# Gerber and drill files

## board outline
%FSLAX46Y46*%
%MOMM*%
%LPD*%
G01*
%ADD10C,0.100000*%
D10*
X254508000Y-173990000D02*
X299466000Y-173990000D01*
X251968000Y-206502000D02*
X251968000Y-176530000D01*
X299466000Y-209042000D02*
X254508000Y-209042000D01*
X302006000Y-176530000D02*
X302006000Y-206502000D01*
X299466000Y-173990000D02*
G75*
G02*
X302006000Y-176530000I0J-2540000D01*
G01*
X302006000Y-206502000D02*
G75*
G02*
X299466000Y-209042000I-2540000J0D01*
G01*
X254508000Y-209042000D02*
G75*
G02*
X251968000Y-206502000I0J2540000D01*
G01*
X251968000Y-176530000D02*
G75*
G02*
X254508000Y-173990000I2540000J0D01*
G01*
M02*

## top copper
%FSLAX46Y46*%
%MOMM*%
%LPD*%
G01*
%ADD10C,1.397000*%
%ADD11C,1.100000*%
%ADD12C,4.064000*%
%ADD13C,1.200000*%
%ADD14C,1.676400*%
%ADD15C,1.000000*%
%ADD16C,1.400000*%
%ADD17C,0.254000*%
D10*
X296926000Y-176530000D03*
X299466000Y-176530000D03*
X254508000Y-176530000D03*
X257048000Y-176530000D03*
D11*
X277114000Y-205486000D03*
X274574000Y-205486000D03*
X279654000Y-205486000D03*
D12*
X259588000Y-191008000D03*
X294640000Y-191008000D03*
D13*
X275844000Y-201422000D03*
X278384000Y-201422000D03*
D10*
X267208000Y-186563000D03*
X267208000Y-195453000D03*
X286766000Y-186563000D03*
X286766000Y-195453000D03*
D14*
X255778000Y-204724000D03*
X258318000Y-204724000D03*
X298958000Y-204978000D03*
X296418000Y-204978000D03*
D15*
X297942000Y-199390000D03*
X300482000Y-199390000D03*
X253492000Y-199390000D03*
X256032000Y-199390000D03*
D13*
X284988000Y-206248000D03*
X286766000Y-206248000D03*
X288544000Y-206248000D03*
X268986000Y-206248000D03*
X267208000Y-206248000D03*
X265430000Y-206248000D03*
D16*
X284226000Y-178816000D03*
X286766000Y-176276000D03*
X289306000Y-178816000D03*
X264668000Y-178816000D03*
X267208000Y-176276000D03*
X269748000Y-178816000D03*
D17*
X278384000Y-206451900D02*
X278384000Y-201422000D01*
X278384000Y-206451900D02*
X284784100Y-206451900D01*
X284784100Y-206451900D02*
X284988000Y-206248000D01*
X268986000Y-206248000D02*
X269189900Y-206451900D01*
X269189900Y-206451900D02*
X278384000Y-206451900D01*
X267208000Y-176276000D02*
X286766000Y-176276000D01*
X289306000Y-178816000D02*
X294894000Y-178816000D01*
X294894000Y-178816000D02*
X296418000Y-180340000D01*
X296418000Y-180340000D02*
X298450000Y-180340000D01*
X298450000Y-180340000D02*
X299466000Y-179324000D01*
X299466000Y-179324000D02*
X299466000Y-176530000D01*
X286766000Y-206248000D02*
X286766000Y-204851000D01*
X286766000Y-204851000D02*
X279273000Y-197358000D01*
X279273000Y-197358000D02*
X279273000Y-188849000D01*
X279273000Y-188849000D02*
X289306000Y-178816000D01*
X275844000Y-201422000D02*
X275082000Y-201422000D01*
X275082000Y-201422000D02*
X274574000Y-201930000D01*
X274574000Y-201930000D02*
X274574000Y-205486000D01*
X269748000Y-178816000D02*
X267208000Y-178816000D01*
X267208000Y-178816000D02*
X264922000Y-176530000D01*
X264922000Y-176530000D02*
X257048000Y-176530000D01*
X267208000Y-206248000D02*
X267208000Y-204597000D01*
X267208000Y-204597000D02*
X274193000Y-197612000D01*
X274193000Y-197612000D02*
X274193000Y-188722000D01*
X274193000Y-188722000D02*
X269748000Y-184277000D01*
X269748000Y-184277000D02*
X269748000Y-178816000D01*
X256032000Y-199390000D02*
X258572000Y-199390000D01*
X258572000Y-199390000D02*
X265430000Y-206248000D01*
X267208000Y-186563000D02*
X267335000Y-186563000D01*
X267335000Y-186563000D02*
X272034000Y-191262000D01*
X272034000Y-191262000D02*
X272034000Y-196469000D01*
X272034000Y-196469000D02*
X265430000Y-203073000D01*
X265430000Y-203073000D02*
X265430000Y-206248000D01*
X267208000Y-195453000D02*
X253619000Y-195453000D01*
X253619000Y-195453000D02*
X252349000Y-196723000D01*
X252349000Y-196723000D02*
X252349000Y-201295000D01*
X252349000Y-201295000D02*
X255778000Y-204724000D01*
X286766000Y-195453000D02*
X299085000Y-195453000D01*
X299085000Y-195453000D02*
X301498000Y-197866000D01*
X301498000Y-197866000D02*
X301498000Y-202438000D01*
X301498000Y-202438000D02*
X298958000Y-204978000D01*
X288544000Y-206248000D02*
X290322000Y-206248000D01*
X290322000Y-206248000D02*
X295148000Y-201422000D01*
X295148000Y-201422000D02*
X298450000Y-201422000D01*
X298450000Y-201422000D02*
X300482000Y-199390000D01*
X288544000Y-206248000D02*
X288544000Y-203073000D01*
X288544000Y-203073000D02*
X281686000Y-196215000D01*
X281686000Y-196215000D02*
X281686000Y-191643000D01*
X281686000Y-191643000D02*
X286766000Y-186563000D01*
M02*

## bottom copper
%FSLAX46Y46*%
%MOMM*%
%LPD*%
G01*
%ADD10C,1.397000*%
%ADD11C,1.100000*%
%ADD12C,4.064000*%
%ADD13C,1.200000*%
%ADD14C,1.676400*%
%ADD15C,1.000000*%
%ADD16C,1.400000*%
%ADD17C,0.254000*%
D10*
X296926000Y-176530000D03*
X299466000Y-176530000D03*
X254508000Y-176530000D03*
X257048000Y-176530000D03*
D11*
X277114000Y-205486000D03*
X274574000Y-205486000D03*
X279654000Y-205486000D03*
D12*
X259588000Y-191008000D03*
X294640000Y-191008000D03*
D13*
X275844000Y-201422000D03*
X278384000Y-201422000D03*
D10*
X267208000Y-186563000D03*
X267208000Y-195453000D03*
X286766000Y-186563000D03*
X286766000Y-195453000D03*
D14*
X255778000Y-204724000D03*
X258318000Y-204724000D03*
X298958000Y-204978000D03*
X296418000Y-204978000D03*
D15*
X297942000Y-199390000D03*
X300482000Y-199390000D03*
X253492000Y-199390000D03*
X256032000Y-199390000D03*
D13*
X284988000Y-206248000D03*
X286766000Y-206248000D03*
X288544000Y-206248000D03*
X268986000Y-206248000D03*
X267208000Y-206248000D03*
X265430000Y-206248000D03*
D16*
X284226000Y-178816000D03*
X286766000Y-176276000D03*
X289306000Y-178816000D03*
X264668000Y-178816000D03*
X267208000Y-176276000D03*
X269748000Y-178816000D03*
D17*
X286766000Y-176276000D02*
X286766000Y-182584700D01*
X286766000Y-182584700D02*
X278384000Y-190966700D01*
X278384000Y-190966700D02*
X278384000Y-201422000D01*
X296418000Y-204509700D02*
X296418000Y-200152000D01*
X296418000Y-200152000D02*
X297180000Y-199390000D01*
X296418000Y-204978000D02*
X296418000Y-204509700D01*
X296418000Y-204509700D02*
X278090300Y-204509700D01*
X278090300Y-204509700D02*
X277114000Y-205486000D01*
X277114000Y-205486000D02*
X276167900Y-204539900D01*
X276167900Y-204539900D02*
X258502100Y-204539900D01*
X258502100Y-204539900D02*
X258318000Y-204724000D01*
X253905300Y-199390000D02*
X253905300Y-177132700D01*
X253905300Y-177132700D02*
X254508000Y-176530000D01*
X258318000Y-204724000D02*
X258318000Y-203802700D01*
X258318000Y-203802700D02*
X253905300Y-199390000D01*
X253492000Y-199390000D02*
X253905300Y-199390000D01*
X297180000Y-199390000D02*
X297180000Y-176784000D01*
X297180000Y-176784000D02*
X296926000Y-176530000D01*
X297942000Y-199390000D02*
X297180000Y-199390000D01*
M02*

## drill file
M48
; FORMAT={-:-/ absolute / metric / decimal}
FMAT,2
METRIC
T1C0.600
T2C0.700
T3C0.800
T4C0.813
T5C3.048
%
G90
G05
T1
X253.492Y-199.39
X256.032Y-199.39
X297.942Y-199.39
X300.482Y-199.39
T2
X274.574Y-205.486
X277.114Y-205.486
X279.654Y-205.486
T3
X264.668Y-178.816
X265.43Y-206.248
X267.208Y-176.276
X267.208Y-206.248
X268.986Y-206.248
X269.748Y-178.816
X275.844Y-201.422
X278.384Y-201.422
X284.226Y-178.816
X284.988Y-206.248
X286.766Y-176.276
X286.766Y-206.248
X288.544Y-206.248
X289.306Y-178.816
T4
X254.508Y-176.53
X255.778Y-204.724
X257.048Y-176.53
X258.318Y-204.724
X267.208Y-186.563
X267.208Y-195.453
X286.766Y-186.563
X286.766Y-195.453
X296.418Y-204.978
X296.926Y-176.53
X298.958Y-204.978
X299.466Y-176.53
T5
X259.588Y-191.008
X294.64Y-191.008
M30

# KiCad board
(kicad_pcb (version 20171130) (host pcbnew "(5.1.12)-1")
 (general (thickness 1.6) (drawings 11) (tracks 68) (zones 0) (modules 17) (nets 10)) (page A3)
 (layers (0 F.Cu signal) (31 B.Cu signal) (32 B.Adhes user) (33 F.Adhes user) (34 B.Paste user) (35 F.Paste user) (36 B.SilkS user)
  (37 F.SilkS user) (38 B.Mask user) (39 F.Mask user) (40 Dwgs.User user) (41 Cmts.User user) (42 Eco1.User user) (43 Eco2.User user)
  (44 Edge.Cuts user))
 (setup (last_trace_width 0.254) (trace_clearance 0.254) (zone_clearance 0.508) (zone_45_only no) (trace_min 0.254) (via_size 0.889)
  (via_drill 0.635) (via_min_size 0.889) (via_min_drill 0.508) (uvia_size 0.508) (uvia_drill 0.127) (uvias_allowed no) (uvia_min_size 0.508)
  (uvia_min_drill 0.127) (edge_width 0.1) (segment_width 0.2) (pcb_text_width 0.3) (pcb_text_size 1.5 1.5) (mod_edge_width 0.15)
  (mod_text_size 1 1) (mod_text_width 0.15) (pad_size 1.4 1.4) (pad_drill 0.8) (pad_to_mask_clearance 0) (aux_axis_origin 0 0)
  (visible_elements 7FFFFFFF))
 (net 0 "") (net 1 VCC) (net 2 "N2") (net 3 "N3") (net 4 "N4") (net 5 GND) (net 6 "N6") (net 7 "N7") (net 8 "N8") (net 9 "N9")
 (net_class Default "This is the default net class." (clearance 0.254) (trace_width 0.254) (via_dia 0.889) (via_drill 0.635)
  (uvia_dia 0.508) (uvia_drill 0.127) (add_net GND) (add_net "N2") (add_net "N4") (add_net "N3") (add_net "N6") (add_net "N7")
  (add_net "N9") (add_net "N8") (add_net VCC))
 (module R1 (layer F.Cu) (at 298.196 176.53) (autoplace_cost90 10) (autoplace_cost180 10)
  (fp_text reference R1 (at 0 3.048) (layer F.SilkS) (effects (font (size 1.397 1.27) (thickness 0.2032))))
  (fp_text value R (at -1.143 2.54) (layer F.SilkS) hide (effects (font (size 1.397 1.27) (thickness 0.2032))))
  (pad 1 thru_hole circle (at -1.27 0) (size 1.397 1.397) (drill 0.8128) (layers *.Cu *.Mask F.SilkS) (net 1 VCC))
  (pad 2 thru_hole circle (at 1.27 0) (size 1.397 1.397) (drill 0.8128) (layers *.Cu *.Mask F.SilkS) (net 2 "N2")))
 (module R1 (layer F.Cu) (at 255.778 176.53) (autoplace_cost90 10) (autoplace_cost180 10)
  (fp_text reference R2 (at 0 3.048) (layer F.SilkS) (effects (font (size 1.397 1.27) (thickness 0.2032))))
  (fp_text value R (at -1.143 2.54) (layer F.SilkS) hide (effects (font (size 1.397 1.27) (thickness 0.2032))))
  (pad 1 thru_hole circle (at -1.27 0) (size 1.397 1.397) (drill 0.8128) (layers *.Cu *.Mask F.SilkS) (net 1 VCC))
  (pad 2 thru_hole circle (at 1.27 0) (size 1.397 1.397) (drill 0.8128) (layers *.Cu *.Mask F.SilkS) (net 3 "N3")))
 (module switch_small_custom (layer F.Cu) (at 277.114 205.486)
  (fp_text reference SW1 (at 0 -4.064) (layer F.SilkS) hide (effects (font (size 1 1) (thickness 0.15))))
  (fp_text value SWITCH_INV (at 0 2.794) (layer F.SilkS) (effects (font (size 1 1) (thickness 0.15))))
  (pad 2 thru_hole circle (at 0 0) (size 1.1 1.1) (drill 0.7) (layers *.Cu *.Mask F.SilkS) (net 1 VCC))
  (pad 1 thru_hole circle (at -2.54 0) (size 1.1 1.1) (drill 0.7) (layers *.Cu *.Mask F.SilkS) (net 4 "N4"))
  (pad 3 thru_hole circle (at 2.54 0) (size 1.1 1.1) (drill 0.7) (layers *.Cu *.Mask F.SilkS)))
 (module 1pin (layer F.Cu) (at 259.588 191.008)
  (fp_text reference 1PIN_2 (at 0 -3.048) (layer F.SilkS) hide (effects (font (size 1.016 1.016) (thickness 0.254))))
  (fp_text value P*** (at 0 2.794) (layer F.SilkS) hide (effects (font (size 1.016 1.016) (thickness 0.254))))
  (pad 1 thru_hole circle (at 0 0) (size 4.064 4.064) (drill 3.048) (layers *.Cu *.Mask F.SilkS)))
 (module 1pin (layer F.Cu) (at 294.64 191.008)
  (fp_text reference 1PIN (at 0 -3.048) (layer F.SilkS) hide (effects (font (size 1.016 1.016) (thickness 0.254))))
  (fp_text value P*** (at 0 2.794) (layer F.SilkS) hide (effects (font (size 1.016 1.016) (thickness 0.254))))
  (pad 1 thru_hole circle (at 0 0) (size 4.064 4.064) (drill 3.048) (layers *.Cu *.Mask F.SilkS)))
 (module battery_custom (layer F.Cu) (at 277.114 201.422)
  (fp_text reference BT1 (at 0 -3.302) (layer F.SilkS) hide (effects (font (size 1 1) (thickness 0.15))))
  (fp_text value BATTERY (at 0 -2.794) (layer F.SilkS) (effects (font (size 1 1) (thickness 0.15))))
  (pad 1 thru_hole circle (at -1.27 0) (size 1.2 1.2) (drill 0.8) (layers *.Cu *.Mask F.SilkS) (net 4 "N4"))
  (pad 2 thru_hole circle (at 1.27 0) (size 1.2 1.2) (drill 0.8) (layers *.Cu *.Mask F.SilkS) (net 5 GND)))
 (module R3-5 (layer F.Cu) (at 267.208 191.008 270)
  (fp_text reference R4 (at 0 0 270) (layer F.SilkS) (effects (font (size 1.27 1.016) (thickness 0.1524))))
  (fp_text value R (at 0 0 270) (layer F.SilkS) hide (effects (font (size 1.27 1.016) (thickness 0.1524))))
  (pad 1 thru_hole circle (at -4.445 0 270) (size 1.397 1.397) (drill 0.8128) (layers *.Cu *.Mask F.SilkS) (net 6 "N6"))
  (pad 2 thru_hole circle (at 4.445 0 270) (size 1.397 1.397) (drill 0.8128) (layers *.Cu *.Mask F.SilkS) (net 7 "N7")))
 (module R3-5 (layer F.Cu) (at 286.766 191.008 270)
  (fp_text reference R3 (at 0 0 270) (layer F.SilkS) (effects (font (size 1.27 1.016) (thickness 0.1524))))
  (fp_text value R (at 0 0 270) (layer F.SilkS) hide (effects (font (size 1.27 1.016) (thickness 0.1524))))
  (pad 1 thru_hole circle (at -4.445 0 270) (size 1.397 1.397) (drill 0.8128) (layers *.Cu *.Mask F.SilkS) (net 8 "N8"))
  (pad 2 thru_hole circle (at 4.445 0 270) (size 1.397 1.397) (drill 0.8128) (layers *.Cu *.Mask F.SilkS) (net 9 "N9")))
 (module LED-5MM (layer F.Cu) (at 257.048 204.724)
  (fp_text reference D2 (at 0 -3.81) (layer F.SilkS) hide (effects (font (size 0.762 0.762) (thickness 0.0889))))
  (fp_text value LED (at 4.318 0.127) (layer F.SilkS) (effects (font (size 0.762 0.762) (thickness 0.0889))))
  (pad 1 thru_hole circle (at -1.27 0) (size 1.6764 1.6764) (drill 0.8128) (layers *.Cu *.Mask F.SilkS) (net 7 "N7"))
  (pad 2 thru_hole circle (at 1.27 0) (size 1.6764 1.6764) (drill 0.8128) (layers *.Cu *.Mask F.SilkS) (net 1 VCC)))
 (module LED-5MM (layer F.Cu) (at 297.688 204.978 180)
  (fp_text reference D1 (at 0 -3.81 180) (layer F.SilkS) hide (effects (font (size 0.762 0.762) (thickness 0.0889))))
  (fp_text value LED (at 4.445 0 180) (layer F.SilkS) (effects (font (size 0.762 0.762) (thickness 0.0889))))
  (pad 1 thru_hole circle (at -1.27 0 180) (size 1.6764 1.6764) (drill 0.8128) (layers *.Cu *.Mask F.SilkS) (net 9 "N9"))
  (pad 2 thru_hole circle (at 1.27 0 180) (size 1.6764 1.6764) (drill 0.8128) (layers *.Cu *.Mask F.SilkS) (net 1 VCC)))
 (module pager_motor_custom (layer F.Cu) (at 299.212 199.39)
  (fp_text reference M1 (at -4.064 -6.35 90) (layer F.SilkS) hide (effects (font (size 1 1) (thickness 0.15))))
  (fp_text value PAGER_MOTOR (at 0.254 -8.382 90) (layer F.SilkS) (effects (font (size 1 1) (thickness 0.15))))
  (pad 1 thru_hole circle (at -1.27 0) (size 1 1) (drill 0.6) (layers *.Cu *.Mask F.SilkS) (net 1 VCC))
  (pad 2 thru_hole circle (at 1.27 0) (size 1 1) (drill 0.6) (layers *.Cu *.Mask F.SilkS) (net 8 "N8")))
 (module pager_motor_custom (layer F.Cu) (at 254.762 199.39)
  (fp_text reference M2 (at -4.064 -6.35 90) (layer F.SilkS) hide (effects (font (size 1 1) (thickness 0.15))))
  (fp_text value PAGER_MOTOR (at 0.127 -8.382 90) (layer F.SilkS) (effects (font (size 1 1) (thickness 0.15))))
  (pad 1 thru_hole circle (at -1.27 0) (size 1 1) (drill 0.6) (layers *.Cu *.Mask F.SilkS) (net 1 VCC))
  (pad 2 thru_hole circle (at 1.27 0) (size 1 1) (drill 0.6) (layers *.Cu *.Mask F.SilkS) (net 6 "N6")))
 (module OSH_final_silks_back (layer F.Cu) (at 277.114 178.943)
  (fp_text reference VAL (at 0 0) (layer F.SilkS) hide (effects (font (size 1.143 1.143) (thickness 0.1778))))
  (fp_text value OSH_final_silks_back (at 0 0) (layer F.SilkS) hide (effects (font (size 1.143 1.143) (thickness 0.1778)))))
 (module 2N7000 (layer F.Cu) (at 286.766 206.248)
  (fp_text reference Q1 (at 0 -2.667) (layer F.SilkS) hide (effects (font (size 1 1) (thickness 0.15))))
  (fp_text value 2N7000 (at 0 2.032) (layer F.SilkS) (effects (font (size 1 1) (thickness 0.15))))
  (pad 1 thru_hole circle (at -1.778 0) (size 1.2 1.2) (drill 0.8) (layers *.Cu *.Mask F.SilkS) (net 5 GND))
  (pad 2 thru_hole circle (at 0 0) (size 1.2 1.2) (drill 0.8) (layers *.Cu *.Mask F.SilkS) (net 2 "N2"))
  (pad 3 thru_hole circle (at 1.778 0) (size 1.2 1.2) (drill 0.8) (layers *.Cu *.Mask F.SilkS) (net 8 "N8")))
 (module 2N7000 (layer F.Cu) (at 267.208 206.248 180)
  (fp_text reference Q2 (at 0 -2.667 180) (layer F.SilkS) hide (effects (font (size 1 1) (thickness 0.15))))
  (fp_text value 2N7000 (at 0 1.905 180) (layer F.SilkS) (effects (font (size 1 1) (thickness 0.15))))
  (pad 1 thru_hole circle (at -1.778 0 180) (size 1.2 1.2) (drill 0.8) (layers *.Cu *.Mask F.SilkS) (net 5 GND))
  (pad 2 thru_hole circle (at 0 0 180) (size 1.2 1.2) (drill 0.8) (layers *.Cu *.Mask F.SilkS) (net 3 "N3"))
  (pad 3 thru_hole circle (at 1.778 0 180) (size 1.2 1.2) (drill 0.8) (layers *.Cu *.Mask F.SilkS) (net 6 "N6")))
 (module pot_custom (layer F.Cu) (at 286.766 178.816)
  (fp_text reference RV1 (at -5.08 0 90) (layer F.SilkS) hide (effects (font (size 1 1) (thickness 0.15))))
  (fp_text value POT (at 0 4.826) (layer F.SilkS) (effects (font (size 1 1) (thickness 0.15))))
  (pad 1 thru_hole circle (at -2.54 0) (size 1.4 1.4) (drill 0.8) (layers *.Cu *.Mask F.SilkS))
  (pad 2 thru_hole circle (at 0 -2.54) (size 1.4 1.4) (drill 0.8) (layers *.Cu *.Mask F.SilkS) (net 5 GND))
  (pad 3 thru_hole circle (at 2.54 0) (size 1.4 1.4) (drill 0.8) (layers *.Cu *.Mask F.SilkS) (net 2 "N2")))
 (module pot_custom (layer F.Cu) (at 267.208 178.816)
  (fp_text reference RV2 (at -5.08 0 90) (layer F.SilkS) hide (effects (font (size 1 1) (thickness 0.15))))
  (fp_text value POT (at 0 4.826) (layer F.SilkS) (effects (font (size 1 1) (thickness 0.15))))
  (pad 1 thru_hole circle (at -2.54 0) (size 1.4 1.4) (drill 0.8) (layers *.Cu *.Mask F.SilkS))
  (pad 2 thru_hole circle (at 0 -2.54) (size 1.4 1.4) (drill 0.8) (layers *.Cu *.Mask F.SilkS) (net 5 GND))
  (pad 3 thru_hole circle (at 2.54 0) (size 1.4 1.4) (drill 0.8) (layers *.Cu *.Mask F.SilkS) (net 3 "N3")))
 (gr_line (start 254.508 173.99) (end 299.466 173.99) (angle 90) (layer Edge.Cuts) (width 0.1))
 (gr_line (start 251.968 206.502) (end 251.968 176.53) (angle 90) (layer Edge.Cuts) (width 0.1))
 (gr_line (start 299.466 209.042) (end 254.508 209.042) (angle 90) (layer Edge.Cuts) (width 0.1))
 (gr_line (start 302.006 176.53) (end 302.006 206.502) (angle 90) (layer Edge.Cuts) (width 0.1))
 (gr_arc (start 299.466 176.53) (end 299.466 173.99) (angle 90) (layer Edge.Cuts) (width 0.1))
 (gr_arc (start 299.466 206.502) (end 302.006 206.502) (angle 90) (layer Edge.Cuts) (width 0.1))
 (gr_arc (start 254.508 206.502) (end 254.508 209.042) (angle 90) (layer Edge.Cuts) (width 0.1))
 (gr_arc (start 254.508 176.53) (end 251.968 176.53) (angle 90) (layer Edge.Cuts) (width 0.1))
 (segment (start 278.384 206.4519) (end 278.384 201.422) (width 0.254) (layer F.Cu) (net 5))
 (segment (start 278.384 206.4519) (end 284.7841 206.4519) (width 0.254) (layer F.Cu) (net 5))
 (segment (start 284.7841 206.4519) (end 284.988 206.248) (width 0.254) (layer F.Cu) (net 5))
 (segment (start 268.986 206.248) (end 269.1899 206.4519) (width 0.254) (layer F.Cu) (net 5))
 (segment (start 269.1899 206.4519) (end 278.384 206.4519) (width 0.254) (layer F.Cu) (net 5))
 (segment (start 286.766 176.276) (end 286.766 182.5847) (width 0.254) (layer B.Cu) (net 5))
 (segment (start 286.766 182.5847) (end 278.384 190.9667) (width 0.254) (layer B.Cu) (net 5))
 (segment (start 278.384 190.9667) (end 278.384 201.422) (width 0.254) (layer B.Cu) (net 5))
 (segment (start 267.208 176.276) (end 286.766 176.276) (width 0.254) (layer F.Cu) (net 5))
 (segment (start 289.306 178.816) (end 294.894 178.816) (width 0.254) (layer F.Cu) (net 2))
 (segment (start 294.894 178.816) (end 296.418 180.34) (width 0.254) (layer F.Cu) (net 2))
 (segment (start 296.418 180.34) (end 298.45 180.34) (width 0.254) (layer F.Cu) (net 2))
 (segment (start 298.45 180.34) (end 299.466 179.324) (width 0.254) (layer F.Cu) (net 2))
 (segment (start 299.466 179.324) (end 299.466 176.53) (width 0.254) (layer F.Cu) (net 2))
 (segment (start 286.766 206.248) (end 286.766 204.851) (width 0.254) (layer F.Cu) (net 2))
 (segment (start 286.766 204.851) (end 279.273 197.358) (width 0.254) (layer F.Cu) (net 2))
 (segment (start 279.273 197.358) (end 279.273 188.849) (width 0.254) (layer F.Cu) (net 2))
 (segment (start 279.273 188.849) (end 289.306 178.816) (width 0.254) (layer F.Cu) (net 2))
 (segment (start 275.844 201.422) (end 275.082 201.422) (width 0.254) (layer F.Cu) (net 4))
 (segment (start 275.082 201.422) (end 274.574 201.93) (width 0.254) (layer F.Cu) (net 4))
 (segment (start 274.574 201.93) (end 274.574 205.486) (width 0.254) (layer F.Cu) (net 4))
 (segment (start 269.748 178.816) (end 267.208 178.816) (width 0.254) (layer F.Cu) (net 3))
 (segment (start 267.208 178.816) (end 264.922 176.53) (width 0.254) (layer F.Cu) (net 3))
 (segment (start 264.922 176.53) (end 257.048 176.53) (width 0.254) (layer F.Cu) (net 3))
 (segment (start 267.208 206.248) (end 267.208 204.597) (width 0.254) (layer F.Cu) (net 3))
 (segment (start 267.208 204.597) (end 274.193 197.612) (width 0.254) (layer F.Cu) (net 3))
 (segment (start 274.193 197.612) (end 274.193 188.722) (width 0.254) (layer F.Cu) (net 3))
 (segment (start 274.193 188.722) (end 269.748 184.277) (width 0.254) (layer F.Cu) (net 3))
 (segment (start 269.748 184.277) (end 269.748 178.816) (width 0.254) (layer F.Cu) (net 3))
 (segment (start 256.032 199.39) (end 258.572 199.39) (width 0.254) (layer F.Cu) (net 6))
 (segment (start 258.572 199.39) (end 265.43 206.248) (width 0.254) (layer F.Cu) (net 6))
 (segment (start 267.208 186.563) (end 267.335 186.563) (width 0.254) (layer F.Cu) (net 6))
 (segment (start 267.335 186.563) (end 272.034 191.262) (width 0.254) (layer F.Cu) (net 6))
 (segment (start 272.034 191.262) (end 272.034 196.469) (width 0.254) (layer F.Cu) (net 6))
 (segment (start 272.034 196.469) (end 265.43 203.073) (width 0.254) (layer F.Cu) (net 6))
 (segment (start 265.43 203.073) (end 265.43 206.248) (width 0.254) (layer F.Cu) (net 6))
 (segment (start 267.208 195.453) (end 253.619 195.453) (width 0.254) (layer F.Cu) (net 7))
 (segment (start 253.619 195.453) (end 252.349 196.723) (width 0.254) (layer F.Cu) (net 7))
 (segment (start 252.349 196.723) (end 252.349 201.295) (width 0.254) (layer F.Cu) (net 7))
 (segment (start 252.349 201.295) (end 255.778 204.724) (width 0.254) (layer F.Cu) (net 7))
 (segment (start 286.766 195.453) (end 299.085 195.453) (width 0.254) (layer F.Cu) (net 9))
 (segment (start 299.085 195.453) (end 301.498 197.866) (width 0.254) (layer F.Cu) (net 9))
 (segment (start 301.498 197.866) (end 301.498 202.438) (width 0.254) (layer F.Cu) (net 9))
 (segment (start 301.498 202.438) (end 298.958 204.978) (width 0.254) (layer F.Cu) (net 9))
 (segment (start 288.544 206.248) (end 290.322 206.248) (width 0.254) (layer F.Cu) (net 8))
 (segment (start 290.322 206.248) (end 295.148 201.422) (width 0.254) (layer F.Cu) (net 8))
 (segment (start 295.148 201.422) (end 298.45 201.422) (width 0.254) (layer F.Cu) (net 8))
 (segment (start 298.45 201.422) (end 300.482 199.39) (width 0.254) (layer F.Cu) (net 8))
 (segment (start 288.544 206.248) (end 288.544 203.073) (width 0.254) (layer F.Cu) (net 8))
 (segment (start 288.544 203.073) (end 281.686 196.215) (width 0.254) (layer F.Cu) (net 8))
 (segment (start 281.686 196.215) (end 281.686 191.643) (width 0.254) (layer F.Cu) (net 8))
 (segment (start 281.686 191.643) (end 286.766 186.563) (width 0.254) (layer F.Cu) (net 8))
 (segment (start 296.418 204.5097) (end 296.418 200.152) (width 0.254) (layer B.Cu) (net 1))
 (segment (start 296.418 200.152) (end 297.18 199.39) (width 0.254) (layer B.Cu) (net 1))
 (segment (start 296.418 204.978) (end 296.418 204.5097) (width 0.254) (layer B.Cu) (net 1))
 (segment (start 296.418 204.5097) (end 278.0903 204.5097) (width 0.254) (layer B.Cu) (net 1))
 (segment (start 278.0903 204.5097) (end 277.114 205.486) (width 0.254) (layer B.Cu) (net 1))
 (segment (start 277.114 205.486) (end 276.1679 204.5399) (width 0.254) (layer B.Cu) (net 1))
 (segment (start 276.1679 204.5399) (end 258.5021 204.5399) (width 0.254) (layer B.Cu) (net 1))
 (segment (start 258.5021 204.5399) (end 258.318 204.724) (width 0.254) (layer B.Cu) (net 1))
 (segment (start 253.9053 199.39) (end 253.9053 177.1327) (width 0.254) (layer B.Cu) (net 1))
 (segment (start 253.9053 177.1327) (end 254.508 176.53) (width 0.254) (layer B.Cu) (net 1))
 (segment (start 258.318 204.724) (end 258.318 203.8027) (width 0.254) (layer B.Cu) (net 1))
 (segment (start 258.318 203.8027) (end 253.9053 199.39) (width 0.254) (layer B.Cu) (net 1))
 (segment (start 253.492 199.39) (end 253.9053 199.39) (width 0.254) (layer B.Cu) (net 1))
 (segment (start 297.18 199.39) (end 297.18 176.784) (width 0.254) (layer B.Cu) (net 1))
 (segment (start 297.18 176.784) (end 296.926 176.53) (width 0.254) (layer B.Cu) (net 1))
 (segment (start 297.942 199.39) (end 297.18 199.39) (width 0.254) (layer B.Cu) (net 1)))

